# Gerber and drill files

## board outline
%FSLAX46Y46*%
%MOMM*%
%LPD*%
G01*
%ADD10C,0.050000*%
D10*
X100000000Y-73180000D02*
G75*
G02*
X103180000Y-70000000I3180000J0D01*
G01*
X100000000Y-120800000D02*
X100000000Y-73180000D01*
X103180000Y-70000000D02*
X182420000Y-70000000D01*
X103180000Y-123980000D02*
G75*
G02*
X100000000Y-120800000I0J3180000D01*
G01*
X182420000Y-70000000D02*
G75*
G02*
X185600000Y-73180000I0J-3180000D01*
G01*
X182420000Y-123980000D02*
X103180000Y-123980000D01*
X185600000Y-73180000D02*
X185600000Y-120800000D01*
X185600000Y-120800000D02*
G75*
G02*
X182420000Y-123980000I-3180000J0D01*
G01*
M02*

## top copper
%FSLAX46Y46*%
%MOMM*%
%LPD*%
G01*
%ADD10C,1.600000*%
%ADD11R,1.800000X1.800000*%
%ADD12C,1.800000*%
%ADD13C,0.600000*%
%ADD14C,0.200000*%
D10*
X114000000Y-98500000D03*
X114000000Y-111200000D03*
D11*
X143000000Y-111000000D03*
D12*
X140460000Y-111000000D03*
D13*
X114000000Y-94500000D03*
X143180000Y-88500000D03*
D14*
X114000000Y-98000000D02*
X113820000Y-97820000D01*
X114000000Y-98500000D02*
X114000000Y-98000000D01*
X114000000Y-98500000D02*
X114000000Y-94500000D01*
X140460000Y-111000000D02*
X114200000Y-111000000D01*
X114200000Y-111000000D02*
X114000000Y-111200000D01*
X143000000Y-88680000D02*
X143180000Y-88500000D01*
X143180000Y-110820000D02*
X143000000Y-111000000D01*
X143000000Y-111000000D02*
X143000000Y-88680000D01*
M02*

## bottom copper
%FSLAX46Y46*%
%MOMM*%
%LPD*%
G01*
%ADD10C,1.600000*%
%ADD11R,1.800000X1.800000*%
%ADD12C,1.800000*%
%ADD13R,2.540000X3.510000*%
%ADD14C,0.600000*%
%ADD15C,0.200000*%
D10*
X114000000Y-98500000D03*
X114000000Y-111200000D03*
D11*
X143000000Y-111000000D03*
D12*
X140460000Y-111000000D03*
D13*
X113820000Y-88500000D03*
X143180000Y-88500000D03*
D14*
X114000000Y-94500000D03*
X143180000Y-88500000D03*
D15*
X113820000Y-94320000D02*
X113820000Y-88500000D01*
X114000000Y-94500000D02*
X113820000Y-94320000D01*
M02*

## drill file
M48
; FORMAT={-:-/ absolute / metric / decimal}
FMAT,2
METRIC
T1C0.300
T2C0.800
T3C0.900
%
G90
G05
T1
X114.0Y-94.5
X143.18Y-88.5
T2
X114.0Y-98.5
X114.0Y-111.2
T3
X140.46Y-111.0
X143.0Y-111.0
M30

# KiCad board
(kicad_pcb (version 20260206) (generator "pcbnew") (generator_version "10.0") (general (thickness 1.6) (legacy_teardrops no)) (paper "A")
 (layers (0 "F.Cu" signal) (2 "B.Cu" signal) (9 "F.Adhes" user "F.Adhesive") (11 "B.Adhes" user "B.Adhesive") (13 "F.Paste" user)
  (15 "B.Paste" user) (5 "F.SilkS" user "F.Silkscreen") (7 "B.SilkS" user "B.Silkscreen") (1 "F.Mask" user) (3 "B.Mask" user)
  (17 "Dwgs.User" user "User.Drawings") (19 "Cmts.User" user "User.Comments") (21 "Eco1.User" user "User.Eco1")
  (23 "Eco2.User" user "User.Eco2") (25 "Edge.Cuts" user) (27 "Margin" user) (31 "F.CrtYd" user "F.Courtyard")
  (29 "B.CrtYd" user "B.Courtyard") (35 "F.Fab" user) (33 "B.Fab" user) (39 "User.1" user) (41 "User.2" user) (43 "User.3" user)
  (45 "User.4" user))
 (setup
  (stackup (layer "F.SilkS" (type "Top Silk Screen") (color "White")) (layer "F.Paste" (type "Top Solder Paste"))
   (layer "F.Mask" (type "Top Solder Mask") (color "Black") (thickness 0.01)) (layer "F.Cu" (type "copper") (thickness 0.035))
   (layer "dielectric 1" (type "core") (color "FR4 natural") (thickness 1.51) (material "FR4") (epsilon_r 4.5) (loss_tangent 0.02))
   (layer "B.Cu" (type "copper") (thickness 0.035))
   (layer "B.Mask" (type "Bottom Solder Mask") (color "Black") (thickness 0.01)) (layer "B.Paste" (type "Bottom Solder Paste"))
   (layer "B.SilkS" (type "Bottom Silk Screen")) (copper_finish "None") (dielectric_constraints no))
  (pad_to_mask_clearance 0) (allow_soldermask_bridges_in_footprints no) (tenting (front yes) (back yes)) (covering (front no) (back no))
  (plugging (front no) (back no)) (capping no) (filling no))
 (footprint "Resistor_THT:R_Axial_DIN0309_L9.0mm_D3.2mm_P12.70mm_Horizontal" (layer "F.Cu") (at 114 98.5 -90)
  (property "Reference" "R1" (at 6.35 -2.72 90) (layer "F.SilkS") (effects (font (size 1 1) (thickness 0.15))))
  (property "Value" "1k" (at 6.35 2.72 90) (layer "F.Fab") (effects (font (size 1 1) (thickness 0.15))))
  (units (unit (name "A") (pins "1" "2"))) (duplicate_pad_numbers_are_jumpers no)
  (pad "1" thru_hole circle (at 0 0 270) (size 1.6 1.6) (drill 0.8) (layers "*.Cu" "*.Mask") (remove_unused_layers no) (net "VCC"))
  (pad "2" thru_hole circle (at 12.7 0 270) (size 1.6 1.6) (drill 0.8) (layers "*.Cu" "*.Mask") (remove_unused_layers no) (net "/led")))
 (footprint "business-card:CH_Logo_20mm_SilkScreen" (layer "F.Cu") (at 170.5 112)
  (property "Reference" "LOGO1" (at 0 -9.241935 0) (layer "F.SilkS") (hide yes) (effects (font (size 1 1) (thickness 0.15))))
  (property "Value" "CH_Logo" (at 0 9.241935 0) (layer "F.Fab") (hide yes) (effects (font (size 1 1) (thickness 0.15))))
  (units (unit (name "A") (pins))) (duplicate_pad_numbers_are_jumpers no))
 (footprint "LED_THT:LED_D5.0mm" (layer "F.Cu") (at 143 111 180)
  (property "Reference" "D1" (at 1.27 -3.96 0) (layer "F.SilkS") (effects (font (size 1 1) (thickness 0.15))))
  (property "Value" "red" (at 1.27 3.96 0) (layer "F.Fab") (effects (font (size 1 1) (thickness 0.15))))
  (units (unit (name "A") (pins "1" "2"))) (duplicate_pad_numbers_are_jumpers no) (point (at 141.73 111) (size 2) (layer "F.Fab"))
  (pad "1" thru_hole rect (at 0 0 180) (size 1.8 1.8) (drill 0.9) (layers "*.Cu" "*.Mask") (remove_unused_layers no) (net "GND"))
  (pad "2" thru_hole circle (at 2.54 0 180) (size 1.8 1.8) (drill 0.9) (layers "*.Cu" "*.Mask") (remove_unused_layers no) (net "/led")))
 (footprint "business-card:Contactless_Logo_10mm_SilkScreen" (layer "F.Cu") (at 177.5 96.764243)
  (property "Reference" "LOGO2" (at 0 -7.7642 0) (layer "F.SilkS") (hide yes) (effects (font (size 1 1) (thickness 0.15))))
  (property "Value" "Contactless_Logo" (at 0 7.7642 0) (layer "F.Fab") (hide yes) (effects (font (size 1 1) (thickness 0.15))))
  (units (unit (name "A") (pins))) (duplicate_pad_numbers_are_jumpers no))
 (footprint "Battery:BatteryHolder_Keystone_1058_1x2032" (layer "B.Cu") (at 128.5 88.5)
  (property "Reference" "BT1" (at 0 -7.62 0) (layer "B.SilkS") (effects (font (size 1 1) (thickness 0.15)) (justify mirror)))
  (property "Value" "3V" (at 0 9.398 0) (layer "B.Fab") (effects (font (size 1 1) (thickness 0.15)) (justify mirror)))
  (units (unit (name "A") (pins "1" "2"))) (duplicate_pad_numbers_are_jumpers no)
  (pad "1" smd rect (at -14.68 0) (size 2.54 3.51) (layers "B.Cu" "B.Mask" "B.Paste") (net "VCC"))
  (pad "2" smd rect (at 14.68 0) (size 2.54 3.51) (layers "B.Cu" "B.Mask" "B.Paste") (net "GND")))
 (gr_arc (start 100 73.18) (mid 100.9314 70.9314) (end 103.18 70) (stroke (width 0.05) (type solid)) (layer "Edge.Cuts"))
 (gr_line (start 100 120.8) (end 100 73.18) (stroke (width 0.05) (type solid)) (layer "Edge.Cuts"))
 (gr_line (start 103.18 70) (end 182.42 70) (stroke (width 0.05) (type solid)) (layer "Edge.Cuts"))
 (gr_arc (start 103.18 123.98) (mid 100.9314 123.0486) (end 100 120.8) (stroke (width 0.05) (type solid)) (layer "Edge.Cuts"))
 (gr_arc (start 182.42 70) (mid 184.6686 70.9314) (end 185.6 73.18) (stroke (width 0.05) (type solid)) (layer "Edge.Cuts"))
 (gr_line (start 182.42 123.98) (end 103.18 123.98) (stroke (width 0.05) (type solid)) (layer "Edge.Cuts"))
 (gr_line (start 185.6 73.18) (end 185.6 120.8) (stroke (width 0.05) (type solid)) (layer "Edge.Cuts"))
 (gr_arc (start 185.6 120.8) (mid 184.6686 123.0486) (end 182.42 123.98) (stroke (width 0.05) (type solid)) (layer "Edge.Cuts"))
 (segment (start 114 98) (end 113.82 97.82) (width 0.2) (layer "F.Cu") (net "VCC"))
 (segment (start 114 98.5) (end 114 98) (width 0.2) (layer "F.Cu") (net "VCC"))
 (segment (start 114 98.5) (end 114 94.5) (width 0.2) (layer "F.Cu") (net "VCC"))
 (via (at 114 94.5) (size 0.6) (drill 0.3) (layers "F.Cu" "B.Cu") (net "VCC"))
 (segment (start 113.82 94.32) (end 113.82 88.5) (width 0.2) (layer "B.Cu") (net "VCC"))
 (segment (start 114 94.5) (end 113.82 94.32) (width 0.2) (layer "B.Cu") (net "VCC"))
 (segment (start 140.46 111) (end 114.2 111) (width 0.2) (layer "F.Cu") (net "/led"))
 (segment (start 114.2 111) (end 114 111.2) (width 0.2) (layer "F.Cu") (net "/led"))
 (segment (start 143 88.68) (end 143.18 88.5) (width 0.2) (layer "F.Cu") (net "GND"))
 (segment (start 143.18 110.82) (end 143 111) (width 0.2) (layer "F.Cu") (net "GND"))
 (segment (start 143 111) (end 143 88.68) (width 0.2) (layer "F.Cu") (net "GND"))
 (via (at 143.18 88.5) (size 0.6) (drill 0.3) (layers "F.Cu" "B.Cu") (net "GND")))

